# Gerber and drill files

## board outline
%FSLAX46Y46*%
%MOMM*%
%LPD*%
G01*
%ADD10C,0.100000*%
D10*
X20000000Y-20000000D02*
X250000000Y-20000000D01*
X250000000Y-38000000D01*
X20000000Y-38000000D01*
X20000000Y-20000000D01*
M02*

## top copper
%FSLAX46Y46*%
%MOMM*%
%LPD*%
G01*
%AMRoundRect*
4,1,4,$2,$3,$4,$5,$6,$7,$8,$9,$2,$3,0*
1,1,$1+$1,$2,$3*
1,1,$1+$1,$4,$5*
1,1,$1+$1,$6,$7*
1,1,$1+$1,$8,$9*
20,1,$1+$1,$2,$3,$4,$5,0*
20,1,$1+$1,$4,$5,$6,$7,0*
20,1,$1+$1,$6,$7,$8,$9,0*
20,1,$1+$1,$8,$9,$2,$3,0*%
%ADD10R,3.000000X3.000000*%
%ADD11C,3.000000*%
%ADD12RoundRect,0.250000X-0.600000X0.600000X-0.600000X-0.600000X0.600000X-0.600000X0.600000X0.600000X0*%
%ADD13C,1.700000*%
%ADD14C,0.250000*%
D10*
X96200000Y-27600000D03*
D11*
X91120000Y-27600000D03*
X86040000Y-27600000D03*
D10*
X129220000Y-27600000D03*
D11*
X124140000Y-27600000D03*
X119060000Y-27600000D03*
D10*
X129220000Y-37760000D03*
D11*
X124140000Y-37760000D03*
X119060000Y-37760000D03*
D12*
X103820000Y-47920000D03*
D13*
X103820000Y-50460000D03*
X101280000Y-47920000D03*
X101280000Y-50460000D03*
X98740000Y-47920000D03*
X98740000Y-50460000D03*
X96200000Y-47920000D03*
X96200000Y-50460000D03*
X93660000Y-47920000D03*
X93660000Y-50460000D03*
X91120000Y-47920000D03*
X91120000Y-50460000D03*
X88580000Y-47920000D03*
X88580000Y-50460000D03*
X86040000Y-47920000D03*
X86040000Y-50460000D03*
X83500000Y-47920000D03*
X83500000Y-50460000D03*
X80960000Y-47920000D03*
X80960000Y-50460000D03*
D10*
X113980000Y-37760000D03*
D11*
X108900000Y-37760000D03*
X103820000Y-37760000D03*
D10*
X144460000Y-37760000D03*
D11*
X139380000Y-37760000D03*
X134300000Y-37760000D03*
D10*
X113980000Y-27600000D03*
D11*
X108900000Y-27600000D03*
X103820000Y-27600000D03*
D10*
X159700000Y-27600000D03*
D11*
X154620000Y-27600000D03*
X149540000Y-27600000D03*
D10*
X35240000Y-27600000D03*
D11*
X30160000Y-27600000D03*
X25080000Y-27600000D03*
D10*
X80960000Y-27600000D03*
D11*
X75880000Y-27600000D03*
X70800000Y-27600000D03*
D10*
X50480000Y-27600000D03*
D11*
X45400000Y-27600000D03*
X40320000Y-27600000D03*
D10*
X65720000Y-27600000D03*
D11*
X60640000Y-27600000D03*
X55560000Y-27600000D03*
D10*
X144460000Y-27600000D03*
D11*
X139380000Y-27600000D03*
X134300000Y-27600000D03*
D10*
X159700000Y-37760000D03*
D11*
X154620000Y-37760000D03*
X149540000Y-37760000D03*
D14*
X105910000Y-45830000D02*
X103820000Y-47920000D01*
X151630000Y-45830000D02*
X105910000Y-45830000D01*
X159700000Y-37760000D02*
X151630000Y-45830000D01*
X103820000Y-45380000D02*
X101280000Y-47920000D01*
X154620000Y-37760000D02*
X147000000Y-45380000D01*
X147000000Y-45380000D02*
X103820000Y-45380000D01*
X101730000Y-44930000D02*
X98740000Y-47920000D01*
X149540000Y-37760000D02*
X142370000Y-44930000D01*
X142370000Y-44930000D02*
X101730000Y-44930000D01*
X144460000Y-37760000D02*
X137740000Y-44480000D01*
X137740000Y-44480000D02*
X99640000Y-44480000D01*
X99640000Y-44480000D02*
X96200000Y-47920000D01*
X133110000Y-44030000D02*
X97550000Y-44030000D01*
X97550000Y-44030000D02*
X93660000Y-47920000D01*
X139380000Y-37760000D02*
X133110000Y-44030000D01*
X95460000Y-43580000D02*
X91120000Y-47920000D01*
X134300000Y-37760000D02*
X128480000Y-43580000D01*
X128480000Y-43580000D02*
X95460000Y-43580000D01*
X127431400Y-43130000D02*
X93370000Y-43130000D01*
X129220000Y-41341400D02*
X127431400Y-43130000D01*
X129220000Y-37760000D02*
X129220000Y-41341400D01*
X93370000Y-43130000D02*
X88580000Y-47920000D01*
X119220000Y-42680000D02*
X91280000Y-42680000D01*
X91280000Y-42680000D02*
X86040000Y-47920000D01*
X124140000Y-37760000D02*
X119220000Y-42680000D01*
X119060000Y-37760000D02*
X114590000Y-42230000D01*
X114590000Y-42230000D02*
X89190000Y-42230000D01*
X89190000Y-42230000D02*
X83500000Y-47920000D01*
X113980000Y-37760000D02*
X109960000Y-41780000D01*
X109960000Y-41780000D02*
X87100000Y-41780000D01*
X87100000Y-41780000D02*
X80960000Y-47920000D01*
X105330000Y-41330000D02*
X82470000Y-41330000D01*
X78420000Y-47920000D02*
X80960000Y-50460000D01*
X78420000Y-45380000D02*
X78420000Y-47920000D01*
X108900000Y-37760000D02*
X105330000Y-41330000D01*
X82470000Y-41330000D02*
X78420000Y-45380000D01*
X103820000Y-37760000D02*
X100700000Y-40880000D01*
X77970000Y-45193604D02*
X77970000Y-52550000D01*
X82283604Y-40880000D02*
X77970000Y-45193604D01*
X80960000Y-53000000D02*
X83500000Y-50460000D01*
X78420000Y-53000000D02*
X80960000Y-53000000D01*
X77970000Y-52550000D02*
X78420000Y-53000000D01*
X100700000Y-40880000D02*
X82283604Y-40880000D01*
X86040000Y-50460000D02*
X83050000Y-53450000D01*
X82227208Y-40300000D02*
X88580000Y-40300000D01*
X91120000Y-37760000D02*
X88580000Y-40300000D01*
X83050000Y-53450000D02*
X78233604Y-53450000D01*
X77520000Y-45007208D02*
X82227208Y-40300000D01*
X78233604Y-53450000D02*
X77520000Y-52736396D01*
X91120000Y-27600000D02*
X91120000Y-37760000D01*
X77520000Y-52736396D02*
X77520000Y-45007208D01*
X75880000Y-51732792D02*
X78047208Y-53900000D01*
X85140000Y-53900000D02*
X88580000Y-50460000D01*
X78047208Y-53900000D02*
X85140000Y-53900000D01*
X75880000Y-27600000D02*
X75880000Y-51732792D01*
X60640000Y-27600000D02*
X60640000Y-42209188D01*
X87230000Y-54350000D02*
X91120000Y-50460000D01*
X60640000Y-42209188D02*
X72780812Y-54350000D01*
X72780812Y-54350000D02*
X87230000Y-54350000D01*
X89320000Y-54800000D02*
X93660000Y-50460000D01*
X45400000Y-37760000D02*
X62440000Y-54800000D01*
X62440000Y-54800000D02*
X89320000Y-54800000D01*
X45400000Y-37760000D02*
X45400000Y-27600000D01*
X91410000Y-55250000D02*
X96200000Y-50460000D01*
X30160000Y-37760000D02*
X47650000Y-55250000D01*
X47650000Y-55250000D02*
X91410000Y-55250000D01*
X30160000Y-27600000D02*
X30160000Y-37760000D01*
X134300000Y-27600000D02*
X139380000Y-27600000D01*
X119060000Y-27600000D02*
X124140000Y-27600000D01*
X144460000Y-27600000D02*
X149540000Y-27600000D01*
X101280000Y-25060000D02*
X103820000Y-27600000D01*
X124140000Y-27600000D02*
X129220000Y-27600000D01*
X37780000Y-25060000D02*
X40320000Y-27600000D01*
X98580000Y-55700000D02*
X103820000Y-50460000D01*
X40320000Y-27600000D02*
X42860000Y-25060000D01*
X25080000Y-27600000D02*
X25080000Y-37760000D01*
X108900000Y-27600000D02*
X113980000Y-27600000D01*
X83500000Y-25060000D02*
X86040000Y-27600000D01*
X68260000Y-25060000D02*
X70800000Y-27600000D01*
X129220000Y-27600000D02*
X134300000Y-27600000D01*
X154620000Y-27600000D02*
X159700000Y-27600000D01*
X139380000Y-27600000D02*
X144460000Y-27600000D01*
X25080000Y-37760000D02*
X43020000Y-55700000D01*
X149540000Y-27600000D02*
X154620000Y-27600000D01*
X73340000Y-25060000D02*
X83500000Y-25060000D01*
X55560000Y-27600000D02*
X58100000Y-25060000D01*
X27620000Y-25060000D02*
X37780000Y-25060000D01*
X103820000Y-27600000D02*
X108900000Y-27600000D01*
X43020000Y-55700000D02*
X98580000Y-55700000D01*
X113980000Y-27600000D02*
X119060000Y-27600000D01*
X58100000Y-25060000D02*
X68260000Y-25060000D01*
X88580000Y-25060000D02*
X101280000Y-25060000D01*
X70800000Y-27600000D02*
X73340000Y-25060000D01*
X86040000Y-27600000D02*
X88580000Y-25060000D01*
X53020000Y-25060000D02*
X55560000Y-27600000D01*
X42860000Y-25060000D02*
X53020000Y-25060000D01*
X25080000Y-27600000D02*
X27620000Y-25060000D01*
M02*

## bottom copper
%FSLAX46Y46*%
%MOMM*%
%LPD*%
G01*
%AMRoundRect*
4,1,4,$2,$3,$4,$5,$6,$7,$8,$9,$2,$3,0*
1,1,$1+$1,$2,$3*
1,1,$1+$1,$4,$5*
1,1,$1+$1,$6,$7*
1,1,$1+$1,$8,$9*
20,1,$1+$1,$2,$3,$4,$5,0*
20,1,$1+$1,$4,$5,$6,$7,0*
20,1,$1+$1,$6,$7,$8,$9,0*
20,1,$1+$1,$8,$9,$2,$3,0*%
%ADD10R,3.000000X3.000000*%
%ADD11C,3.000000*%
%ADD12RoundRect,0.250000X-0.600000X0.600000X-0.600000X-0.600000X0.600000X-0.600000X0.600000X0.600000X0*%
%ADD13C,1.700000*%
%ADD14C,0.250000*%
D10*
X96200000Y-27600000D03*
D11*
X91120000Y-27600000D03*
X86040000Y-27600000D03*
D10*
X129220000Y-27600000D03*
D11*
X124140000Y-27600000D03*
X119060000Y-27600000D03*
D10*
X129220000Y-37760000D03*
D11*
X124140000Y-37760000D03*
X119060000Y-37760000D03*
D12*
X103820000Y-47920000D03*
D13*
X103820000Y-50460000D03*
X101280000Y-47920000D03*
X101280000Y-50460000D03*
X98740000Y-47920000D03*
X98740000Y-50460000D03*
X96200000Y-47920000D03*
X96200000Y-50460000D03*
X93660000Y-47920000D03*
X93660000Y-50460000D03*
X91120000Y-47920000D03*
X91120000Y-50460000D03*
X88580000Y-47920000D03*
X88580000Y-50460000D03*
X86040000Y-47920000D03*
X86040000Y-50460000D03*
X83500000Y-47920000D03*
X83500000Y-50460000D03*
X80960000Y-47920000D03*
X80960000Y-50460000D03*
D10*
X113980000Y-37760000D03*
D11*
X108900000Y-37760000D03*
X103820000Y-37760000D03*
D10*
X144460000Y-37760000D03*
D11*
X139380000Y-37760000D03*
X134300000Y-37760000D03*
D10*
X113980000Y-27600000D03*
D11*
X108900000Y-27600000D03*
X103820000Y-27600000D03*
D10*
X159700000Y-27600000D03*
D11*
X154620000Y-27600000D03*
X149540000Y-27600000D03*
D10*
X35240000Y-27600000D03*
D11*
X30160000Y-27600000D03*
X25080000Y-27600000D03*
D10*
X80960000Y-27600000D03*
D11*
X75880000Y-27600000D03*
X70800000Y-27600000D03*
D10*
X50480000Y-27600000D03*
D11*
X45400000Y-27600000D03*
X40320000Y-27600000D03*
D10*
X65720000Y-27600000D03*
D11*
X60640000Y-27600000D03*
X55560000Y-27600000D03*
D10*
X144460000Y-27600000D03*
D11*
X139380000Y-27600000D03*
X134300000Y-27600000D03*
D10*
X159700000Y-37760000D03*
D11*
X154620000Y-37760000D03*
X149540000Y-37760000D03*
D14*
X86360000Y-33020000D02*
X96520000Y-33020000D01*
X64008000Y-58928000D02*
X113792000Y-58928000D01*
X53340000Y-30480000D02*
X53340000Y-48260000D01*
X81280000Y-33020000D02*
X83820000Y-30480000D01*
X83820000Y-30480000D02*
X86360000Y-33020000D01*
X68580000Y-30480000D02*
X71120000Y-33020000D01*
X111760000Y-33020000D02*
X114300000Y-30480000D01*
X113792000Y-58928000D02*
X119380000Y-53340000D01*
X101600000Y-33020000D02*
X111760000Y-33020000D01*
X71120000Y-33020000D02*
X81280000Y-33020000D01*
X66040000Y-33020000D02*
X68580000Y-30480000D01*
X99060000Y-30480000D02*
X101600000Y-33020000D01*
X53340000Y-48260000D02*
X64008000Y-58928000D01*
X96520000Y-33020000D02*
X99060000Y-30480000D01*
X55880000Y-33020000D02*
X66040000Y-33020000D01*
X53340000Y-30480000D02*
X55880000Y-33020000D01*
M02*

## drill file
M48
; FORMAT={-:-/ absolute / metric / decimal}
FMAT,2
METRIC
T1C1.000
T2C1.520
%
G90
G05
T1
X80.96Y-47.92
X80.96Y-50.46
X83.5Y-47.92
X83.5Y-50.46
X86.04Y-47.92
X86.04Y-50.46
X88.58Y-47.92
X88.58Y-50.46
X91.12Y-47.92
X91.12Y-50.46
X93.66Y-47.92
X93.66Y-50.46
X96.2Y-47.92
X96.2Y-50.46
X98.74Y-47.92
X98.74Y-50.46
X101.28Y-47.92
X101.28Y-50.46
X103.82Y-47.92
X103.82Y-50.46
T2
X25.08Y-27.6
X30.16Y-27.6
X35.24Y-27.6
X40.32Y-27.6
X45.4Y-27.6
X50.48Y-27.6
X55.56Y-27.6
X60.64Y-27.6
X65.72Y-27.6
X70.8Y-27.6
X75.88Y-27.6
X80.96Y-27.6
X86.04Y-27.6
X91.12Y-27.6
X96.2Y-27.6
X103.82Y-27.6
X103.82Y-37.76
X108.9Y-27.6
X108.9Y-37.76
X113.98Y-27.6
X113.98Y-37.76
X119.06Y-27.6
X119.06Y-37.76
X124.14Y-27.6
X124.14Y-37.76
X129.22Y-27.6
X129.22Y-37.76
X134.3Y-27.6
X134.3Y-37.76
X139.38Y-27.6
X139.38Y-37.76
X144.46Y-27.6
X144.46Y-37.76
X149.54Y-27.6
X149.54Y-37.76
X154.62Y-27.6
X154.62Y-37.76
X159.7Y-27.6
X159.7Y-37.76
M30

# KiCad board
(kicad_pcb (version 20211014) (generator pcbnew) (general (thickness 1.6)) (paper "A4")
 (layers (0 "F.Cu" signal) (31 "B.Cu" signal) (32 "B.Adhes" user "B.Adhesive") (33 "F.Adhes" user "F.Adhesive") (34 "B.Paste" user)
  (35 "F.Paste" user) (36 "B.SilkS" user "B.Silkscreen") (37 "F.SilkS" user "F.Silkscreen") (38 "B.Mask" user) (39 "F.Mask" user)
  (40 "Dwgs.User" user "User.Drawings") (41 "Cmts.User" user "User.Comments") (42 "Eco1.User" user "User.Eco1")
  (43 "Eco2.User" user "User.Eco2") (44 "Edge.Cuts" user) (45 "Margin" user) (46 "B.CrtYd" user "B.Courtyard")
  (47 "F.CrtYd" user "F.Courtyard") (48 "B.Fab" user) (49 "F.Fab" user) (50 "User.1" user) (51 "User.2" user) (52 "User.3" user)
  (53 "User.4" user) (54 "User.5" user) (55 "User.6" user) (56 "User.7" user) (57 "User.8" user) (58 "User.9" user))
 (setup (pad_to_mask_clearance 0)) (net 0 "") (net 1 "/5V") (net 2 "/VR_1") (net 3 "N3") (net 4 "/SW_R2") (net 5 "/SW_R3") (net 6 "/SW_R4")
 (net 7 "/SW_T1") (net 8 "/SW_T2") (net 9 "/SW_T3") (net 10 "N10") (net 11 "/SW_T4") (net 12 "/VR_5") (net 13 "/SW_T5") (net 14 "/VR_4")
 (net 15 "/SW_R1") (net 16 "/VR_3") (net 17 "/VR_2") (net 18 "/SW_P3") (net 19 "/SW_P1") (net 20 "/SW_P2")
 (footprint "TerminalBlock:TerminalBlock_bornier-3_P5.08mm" (layer "F.Cu") (at 96.2 27.6 180)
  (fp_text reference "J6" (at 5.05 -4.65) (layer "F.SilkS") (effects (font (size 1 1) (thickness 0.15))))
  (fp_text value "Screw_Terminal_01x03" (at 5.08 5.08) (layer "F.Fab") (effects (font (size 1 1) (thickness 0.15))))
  (pad "1" thru_hole rect (at 0 0 180) (size 3 3) (drill 1.52) (layers *.Cu *.Mask) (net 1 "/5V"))
  (pad "2" thru_hole circle (at 5.08 0 180) (size 3 3) (drill 1.52) (layers *.Cu *.Mask) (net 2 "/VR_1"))
  (pad "3" thru_hole circle (at 10.16 0 180) (size 3 3) (drill 1.52) (layers *.Cu *.Mask) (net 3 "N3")))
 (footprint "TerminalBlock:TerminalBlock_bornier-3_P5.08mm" (layer "F.Cu") (at 129.22 27.6 180)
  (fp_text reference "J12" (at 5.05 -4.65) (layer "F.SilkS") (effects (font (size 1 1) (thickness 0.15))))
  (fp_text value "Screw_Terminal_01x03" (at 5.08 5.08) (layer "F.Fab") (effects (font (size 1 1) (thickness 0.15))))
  (pad "1" thru_hole rect (at 0 0 180) (size 3 3) (drill 1.52) (layers *.Cu *.Mask) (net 3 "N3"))
  (pad "2" thru_hole circle (at 5.08 0 180) (size 3 3) (drill 1.52) (layers *.Cu *.Mask) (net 3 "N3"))
  (pad "3" thru_hole circle (at 10.16 0 180) (size 3 3) (drill 1.52) (layers *.Cu *.Mask) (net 3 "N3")))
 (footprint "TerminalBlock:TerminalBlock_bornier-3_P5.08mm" (layer "F.Cu") (at 129.22 37.76 180)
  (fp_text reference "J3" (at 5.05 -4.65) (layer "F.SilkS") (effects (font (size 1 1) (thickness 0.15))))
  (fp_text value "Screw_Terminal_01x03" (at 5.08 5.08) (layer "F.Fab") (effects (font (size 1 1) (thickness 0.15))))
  (pad "1" thru_hole rect (at 0 0 180) (size 3 3) (drill 1.52) (layers *.Cu *.Mask) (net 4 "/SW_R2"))
  (pad "2" thru_hole circle (at 5.08 0 180) (size 3 3) (drill 1.52) (layers *.Cu *.Mask) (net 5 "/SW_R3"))
  (pad "3" thru_hole circle (at 10.16 0 180) (size 3 3) (drill 1.52) (layers *.Cu *.Mask) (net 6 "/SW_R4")))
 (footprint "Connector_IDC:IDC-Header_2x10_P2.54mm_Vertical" (layer "F.Cu") (at 103.82 47.92 -90)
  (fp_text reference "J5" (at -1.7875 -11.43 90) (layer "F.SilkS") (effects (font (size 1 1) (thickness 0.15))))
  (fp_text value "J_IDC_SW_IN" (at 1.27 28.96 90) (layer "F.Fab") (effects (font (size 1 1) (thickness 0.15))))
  (pad "1" thru_hole roundrect (at 0 0 270) (size 1.7 1.7) (drill 1) (layers *.Cu *.Mask) (roundrect_rratio 0.147059) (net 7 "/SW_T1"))
  (pad "2" thru_hole circle (at 2.54 0 270) (size 1.7 1.7) (drill 1) (layers *.Cu *.Mask) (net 3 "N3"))
  (pad "3" thru_hole circle (at 0 2.54 270) (size 1.7 1.7) (drill 1) (layers *.Cu *.Mask) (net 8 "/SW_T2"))
  (pad "4" thru_hole circle (at 2.54 2.54 270) (size 1.7 1.7) (drill 1) (layers *.Cu *.Mask) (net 1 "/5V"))
  (pad "5" thru_hole circle (at 0 5.08 270) (size 1.7 1.7) (drill 1) (layers *.Cu *.Mask) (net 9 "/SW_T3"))
  (pad "6" thru_hole circle (at 2.54 5.08 270) (size 1.7 1.7) (drill 1) (layers *.Cu *.Mask) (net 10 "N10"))
  (pad "7" thru_hole circle (at 0 7.62 270) (size 1.7 1.7) (drill 1) (layers *.Cu *.Mask) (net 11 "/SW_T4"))
  (pad "8" thru_hole circle (at 2.54 7.62 270) (size 1.7 1.7) (drill 1) (layers *.Cu *.Mask) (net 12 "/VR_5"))
  (pad "9" thru_hole circle (at 0 10.16 270) (size 1.7 1.7) (drill 1) (layers *.Cu *.Mask) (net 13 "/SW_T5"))
  (pad "10" thru_hole circle (at 2.54 10.16 270) (size 1.7 1.7) (drill 1) (layers *.Cu *.Mask) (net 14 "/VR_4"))
  (pad "11" thru_hole circle (at 0 12.7 270) (size 1.7 1.7) (drill 1) (layers *.Cu *.Mask) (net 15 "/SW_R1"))
  (pad "12" thru_hole circle (at 2.54 12.7 270) (size 1.7 1.7) (drill 1) (layers *.Cu *.Mask) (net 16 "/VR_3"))
  (pad "13" thru_hole circle (at 0 15.24 270) (size 1.7 1.7) (drill 1) (layers *.Cu *.Mask) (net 4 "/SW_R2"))
  (pad "14" thru_hole circle (at 2.54 15.24 270) (size 1.7 1.7) (drill 1) (layers *.Cu *.Mask) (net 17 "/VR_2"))
  (pad "15" thru_hole circle (at 0 17.78 270) (size 1.7 1.7) (drill 1) (layers *.Cu *.Mask) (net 5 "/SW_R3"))
  (pad "16" thru_hole circle (at 2.54 17.78 270) (size 1.7 1.7) (drill 1) (layers *.Cu *.Mask) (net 2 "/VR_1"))
  (pad "17" thru_hole circle (at 0 20.32 270) (size 1.7 1.7) (drill 1) (layers *.Cu *.Mask) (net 6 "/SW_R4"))
  (pad "18" thru_hole circle (at 2.54 20.32 270) (size 1.7 1.7) (drill 1) (layers *.Cu *.Mask) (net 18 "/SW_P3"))
  (pad "19" thru_hole circle (at 0 22.86 270) (size 1.7 1.7) (drill 1) (layers *.Cu *.Mask) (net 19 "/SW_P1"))
  (pad "20" thru_hole circle (at 2.54 22.86 270) (size 1.7 1.7) (drill 1) (layers *.Cu *.Mask) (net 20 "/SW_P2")))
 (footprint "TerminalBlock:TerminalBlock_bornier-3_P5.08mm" (layer "F.Cu") (at 113.98 37.76 180)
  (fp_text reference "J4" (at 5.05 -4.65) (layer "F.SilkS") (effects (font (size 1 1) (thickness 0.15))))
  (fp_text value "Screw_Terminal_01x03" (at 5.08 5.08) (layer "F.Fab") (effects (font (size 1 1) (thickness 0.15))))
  (pad "1" thru_hole rect (at 0 0 180) (size 3 3) (drill 1.52) (layers *.Cu *.Mask) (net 19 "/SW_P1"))
  (pad "2" thru_hole circle (at 5.08 0 180) (size 3 3) (drill 1.52) (layers *.Cu *.Mask) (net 20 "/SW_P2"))
  (pad "3" thru_hole circle (at 10.16 0 180) (size 3 3) (drill 1.52) (layers *.Cu *.Mask) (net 18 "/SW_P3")))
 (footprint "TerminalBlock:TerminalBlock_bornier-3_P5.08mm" (layer "F.Cu") (at 144.46 37.76 180)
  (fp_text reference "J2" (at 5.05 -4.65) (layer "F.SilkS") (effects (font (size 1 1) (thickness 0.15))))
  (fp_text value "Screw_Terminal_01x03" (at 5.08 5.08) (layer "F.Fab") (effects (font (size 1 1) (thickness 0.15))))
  (pad "1" thru_hole rect (at 0 0 180) (size 3 3) (drill 1.52) (layers *.Cu *.Mask) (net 11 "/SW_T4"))
  (pad "2" thru_hole circle (at 5.08 0 180) (size 3 3) (drill 1.52) (layers *.Cu *.Mask) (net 13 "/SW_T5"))
  (pad "3" thru_hole circle (at 10.16 0 180) (size 3 3) (drill 1.52) (layers *.Cu *.Mask) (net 15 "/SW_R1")))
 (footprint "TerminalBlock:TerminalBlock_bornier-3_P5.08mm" (layer "F.Cu") (at 113.98 27.6 180)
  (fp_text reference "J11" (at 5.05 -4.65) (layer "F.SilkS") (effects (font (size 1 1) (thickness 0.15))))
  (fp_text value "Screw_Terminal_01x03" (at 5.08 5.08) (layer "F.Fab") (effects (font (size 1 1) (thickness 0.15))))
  (pad "1" thru_hole rect (at 0 0 180) (size 3 3) (drill 1.52) (layers *.Cu *.Mask) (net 3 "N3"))
  (pad "2" thru_hole circle (at 5.08 0 180) (size 3 3) (drill 1.52) (layers *.Cu *.Mask) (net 3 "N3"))
  (pad "3" thru_hole circle (at 10.16 0 180) (size 3 3) (drill 1.52) (layers *.Cu *.Mask) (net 3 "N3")))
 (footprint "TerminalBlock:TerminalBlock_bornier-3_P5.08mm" (layer "F.Cu") (at 159.7 27.6 180)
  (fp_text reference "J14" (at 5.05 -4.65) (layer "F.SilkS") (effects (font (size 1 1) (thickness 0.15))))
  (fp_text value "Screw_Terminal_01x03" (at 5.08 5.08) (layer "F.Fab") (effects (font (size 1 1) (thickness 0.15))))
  (pad "1" thru_hole rect (at 0 0 180) (size 3 3) (drill 1.52) (layers *.Cu *.Mask) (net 3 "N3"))
  (pad "2" thru_hole circle (at 5.08 0 180) (size 3 3) (drill 1.52) (layers *.Cu *.Mask) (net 3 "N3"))
  (pad "3" thru_hole circle (at 10.16 0 180) (size 3 3) (drill 1.52) (layers *.Cu *.Mask) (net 3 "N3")))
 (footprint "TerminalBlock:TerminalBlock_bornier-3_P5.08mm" (layer "F.Cu") (at 35.24 27.6 180)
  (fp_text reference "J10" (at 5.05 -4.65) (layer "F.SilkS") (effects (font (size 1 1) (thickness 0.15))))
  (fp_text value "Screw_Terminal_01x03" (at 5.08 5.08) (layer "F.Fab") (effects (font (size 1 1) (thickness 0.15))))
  (pad "1" thru_hole rect (at 0 0 180) (size 3 3) (drill 1.52) (layers *.Cu *.Mask) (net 1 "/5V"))
  (pad "2" thru_hole circle (at 5.08 0 180) (size 3 3) (drill 1.52) (layers *.Cu *.Mask) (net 12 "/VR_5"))
  (pad "3" thru_hole circle (at 10.16 0 180) (size 3 3) (drill 1.52) (layers *.Cu *.Mask) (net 3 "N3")))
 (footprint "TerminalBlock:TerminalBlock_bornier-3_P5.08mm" (layer "F.Cu") (at 80.96 27.6 180)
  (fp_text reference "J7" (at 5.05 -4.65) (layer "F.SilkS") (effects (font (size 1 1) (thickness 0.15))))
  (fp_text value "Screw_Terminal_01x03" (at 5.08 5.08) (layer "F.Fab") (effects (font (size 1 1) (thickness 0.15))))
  (pad "1" thru_hole rect (at 0 0 180) (size 3 3) (drill 1.52) (layers *.Cu *.Mask) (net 1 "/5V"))
  (pad "2" thru_hole circle (at 5.08 0 180) (size 3 3) (drill 1.52) (layers *.Cu *.Mask) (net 17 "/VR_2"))
  (pad "3" thru_hole circle (at 10.16 0 180) (size 3 3) (drill 1.52) (layers *.Cu *.Mask) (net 3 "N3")))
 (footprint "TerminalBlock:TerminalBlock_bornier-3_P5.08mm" (layer "F.Cu") (at 50.48 27.6 180)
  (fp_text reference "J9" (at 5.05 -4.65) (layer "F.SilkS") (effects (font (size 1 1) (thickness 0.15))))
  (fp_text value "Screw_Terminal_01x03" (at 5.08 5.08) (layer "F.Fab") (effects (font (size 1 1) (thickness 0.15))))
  (pad "1" thru_hole rect (at 0 0 180) (size 3 3) (drill 1.52) (layers *.Cu *.Mask) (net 1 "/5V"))
  (pad "2" thru_hole circle (at 5.08 0 180) (size 3 3) (drill 1.52) (layers *.Cu *.Mask) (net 14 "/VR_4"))
  (pad "3" thru_hole circle (at 10.16 0 180) (size 3 3) (drill 1.52) (layers *.Cu *.Mask) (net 3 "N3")))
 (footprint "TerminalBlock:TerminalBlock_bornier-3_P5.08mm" (layer "F.Cu") (at 65.72 27.6 180)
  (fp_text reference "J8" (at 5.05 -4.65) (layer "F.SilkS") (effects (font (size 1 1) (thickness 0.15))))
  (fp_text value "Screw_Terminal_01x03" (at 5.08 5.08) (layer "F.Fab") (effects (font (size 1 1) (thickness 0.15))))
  (pad "1" thru_hole rect (at 0 0 180) (size 3 3) (drill 1.52) (layers *.Cu *.Mask) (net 1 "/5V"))
  (pad "2" thru_hole circle (at 5.08 0 180) (size 3 3) (drill 1.52) (layers *.Cu *.Mask) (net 16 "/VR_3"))
  (pad "3" thru_hole circle (at 10.16 0 180) (size 3 3) (drill 1.52) (layers *.Cu *.Mask) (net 3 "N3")))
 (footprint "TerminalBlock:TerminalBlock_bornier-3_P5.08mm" (layer "F.Cu") (at 144.46 27.6 180)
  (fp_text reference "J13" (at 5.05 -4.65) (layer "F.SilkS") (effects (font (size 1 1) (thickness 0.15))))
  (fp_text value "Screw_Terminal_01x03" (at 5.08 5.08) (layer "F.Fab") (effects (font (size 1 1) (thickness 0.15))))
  (pad "1" thru_hole rect (at 0 0 180) (size 3 3) (drill 1.52) (layers *.Cu *.Mask) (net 3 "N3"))
  (pad "2" thru_hole circle (at 5.08 0 180) (size 3 3) (drill 1.52) (layers *.Cu *.Mask) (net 3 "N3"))
  (pad "3" thru_hole circle (at 10.16 0 180) (size 3 3) (drill 1.52) (layers *.Cu *.Mask) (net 3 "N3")))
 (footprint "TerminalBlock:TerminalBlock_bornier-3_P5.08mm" (layer "F.Cu") (at 159.7 37.76 180)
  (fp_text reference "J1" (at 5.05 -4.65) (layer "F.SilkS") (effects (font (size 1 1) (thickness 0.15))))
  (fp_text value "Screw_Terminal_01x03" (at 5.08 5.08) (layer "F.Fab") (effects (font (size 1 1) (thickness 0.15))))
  (pad "1" thru_hole rect (at 0 0 180) (size 3 3) (drill 1.52) (layers *.Cu *.Mask) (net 7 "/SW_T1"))
  (pad "2" thru_hole circle (at 5.08 0 180) (size 3 3) (drill 1.52) (layers *.Cu *.Mask) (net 8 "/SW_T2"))
  (pad "3" thru_hole circle (at 10.16 0 180) (size 3 3) (drill 1.52) (layers *.Cu *.Mask) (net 9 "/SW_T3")))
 (gr_rect (start 20 20) (end 250 38) (layer "Edge.Cuts") (width 0.1) (fill none))
 (segment (start 105.91 45.83) (end 103.82 47.92) (width 0.25) (layer "F.Cu") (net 7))
 (segment (start 151.63 45.83) (end 105.91 45.83) (width 0.25) (layer "F.Cu") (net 7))
 (segment (start 159.7 37.76) (end 151.63 45.83) (width 0.25) (layer "F.Cu") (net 7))
 (segment (start 103.82 45.38) (end 101.28 47.92) (width 0.25) (layer "F.Cu") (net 8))
 (segment (start 154.62 37.76) (end 147 45.38) (width 0.25) (layer "F.Cu") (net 8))
 (segment (start 147 45.38) (end 103.82 45.38) (width 0.25) (layer "F.Cu") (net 8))
 (segment (start 101.73 44.93) (end 98.74 47.92) (width 0.25) (layer "F.Cu") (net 9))
 (segment (start 149.54 37.76) (end 142.37 44.93) (width 0.25) (layer "F.Cu") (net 9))
 (segment (start 142.37 44.93) (end 101.73 44.93) (width 0.25) (layer "F.Cu") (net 9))
 (segment (start 144.46 37.76) (end 137.74 44.48) (width 0.25) (layer "F.Cu") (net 11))
 (segment (start 137.74 44.48) (end 99.64 44.48) (width 0.25) (layer "F.Cu") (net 11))
 (segment (start 99.64 44.48) (end 96.2 47.92) (width 0.25) (layer "F.Cu") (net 11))
 (segment (start 133.11 44.03) (end 97.55 44.03) (width 0.25) (layer "F.Cu") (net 13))
 (segment (start 97.55 44.03) (end 93.66 47.92) (width 0.25) (layer "F.Cu") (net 13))
 (segment (start 139.38 37.76) (end 133.11 44.03) (width 0.25) (layer "F.Cu") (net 13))
 (segment (start 95.46 43.58) (end 91.12 47.92) (width 0.25) (layer "F.Cu") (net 15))
 (segment (start 134.3 37.76) (end 128.48 43.58) (width 0.25) (layer "F.Cu") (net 15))
 (segment (start 128.48 43.58) (end 95.46 43.58) (width 0.25) (layer "F.Cu") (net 15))
 (segment (start 127.4314 43.13) (end 93.37 43.13) (width 0.25) (layer "F.Cu") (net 4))
 (segment (start 129.22 41.3414) (end 127.4314 43.13) (width 0.25) (layer "F.Cu") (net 4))
 (segment (start 129.22 37.76) (end 129.22 41.3414) (width 0.25) (layer "F.Cu") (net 4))
 (segment (start 93.37 43.13) (end 88.58 47.92) (width 0.25) (layer "F.Cu") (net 4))
 (segment (start 119.22 42.68) (end 91.28 42.68) (width 0.25) (layer "F.Cu") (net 5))
 (segment (start 91.28 42.68) (end 86.04 47.92) (width 0.25) (layer "F.Cu") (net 5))
 (segment (start 124.14 37.76) (end 119.22 42.68) (width 0.25) (layer "F.Cu") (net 5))
 (segment (start 119.06 37.76) (end 114.59 42.23) (width 0.25) (layer "F.Cu") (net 6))
 (segment (start 114.59 42.23) (end 89.19 42.23) (width 0.25) (layer "F.Cu") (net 6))
 (segment (start 89.19 42.23) (end 83.5 47.92) (width 0.25) (layer "F.Cu") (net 6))
 (segment (start 113.98 37.76) (end 109.96 41.78) (width 0.25) (layer "F.Cu") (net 19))
 (segment (start 109.96 41.78) (end 87.1 41.78) (width 0.25) (layer "F.Cu") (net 19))
 (segment (start 87.1 41.78) (end 80.96 47.92) (width 0.25) (layer "F.Cu") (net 19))
 (segment (start 105.33 41.33) (end 82.47 41.33) (width 0.25) (layer "F.Cu") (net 20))
 (segment (start 78.42 47.92) (end 80.96 50.46) (width 0.25) (layer "F.Cu") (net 20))
 (segment (start 78.42 45.38) (end 78.42 47.92) (width 0.25) (layer "F.Cu") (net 20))
 (segment (start 108.9 37.76) (end 105.33 41.33) (width 0.25) (layer "F.Cu") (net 20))
 (segment (start 82.47 41.33) (end 78.42 45.38) (width 0.25) (layer "F.Cu") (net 20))
 (segment (start 103.82 37.76) (end 100.7 40.88) (width 0.25) (layer "F.Cu") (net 18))
 (segment (start 77.97 45.193604) (end 77.97 52.55) (width 0.25) (layer "F.Cu") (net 18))
 (segment (start 82.283604 40.88) (end 77.97 45.193604) (width 0.25) (layer "F.Cu") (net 18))
 (segment (start 80.96 53) (end 83.5 50.46) (width 0.25) (layer "F.Cu") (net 18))
 (segment (start 78.42 53) (end 80.96 53) (width 0.25) (layer "F.Cu") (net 18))
 (segment (start 77.97 52.55) (end 78.42 53) (width 0.25) (layer "F.Cu") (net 18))
 (segment (start 100.7 40.88) (end 82.283604 40.88) (width 0.25) (layer "F.Cu") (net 18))
 (segment (start 86.04 50.46) (end 83.05 53.45) (width 0.25) (layer "F.Cu") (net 2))
 (segment (start 82.227208 40.3) (end 88.58 40.3) (width 0.25) (layer "F.Cu") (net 2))
 (segment (start 91.12 37.76) (end 88.58 40.3) (width 0.25) (layer "F.Cu") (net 2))
 (segment (start 83.05 53.45) (end 78.233604 53.45) (width 0.25) (layer "F.Cu") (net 2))
 (segment (start 77.52 45.007208) (end 82.227208 40.3) (width 0.25) (layer "F.Cu") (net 2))
 (segment (start 78.233604 53.45) (end 77.52 52.736396) (width 0.25) (layer "F.Cu") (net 2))
 (segment (start 91.12 27.6) (end 91.12 37.76) (width 0.25) (layer "F.Cu") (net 2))
 (segment (start 77.52 52.736396) (end 77.52 45.007208) (width 0.25) (layer "F.Cu") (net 2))
 (segment (start 75.88 51.732792) (end 78.047208 53.9) (width 0.25) (layer "F.Cu") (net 17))
 (segment (start 85.14 53.9) (end 88.58 50.46) (width 0.25) (layer "F.Cu") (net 17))
 (segment (start 78.047208 53.9) (end 85.14 53.9) (width 0.25) (layer "F.Cu") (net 17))
 (segment (start 75.88 27.6) (end 75.88 51.732792) (width 0.25) (layer "F.Cu") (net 17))
 (segment (start 60.64 27.6) (end 60.64 42.209188) (width 0.25) (layer "F.Cu") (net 16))
 (segment (start 87.23 54.35) (end 91.12 50.46) (width 0.25) (layer "F.Cu") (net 16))
 (segment (start 60.64 42.209188) (end 72.780812 54.35) (width 0.25) (layer "F.Cu") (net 16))
 (segment (start 72.780812 54.35) (end 87.23 54.35) (width 0.25) (layer "F.Cu") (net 16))
 (segment (start 89.32 54.8) (end 93.66 50.46) (width 0.25) (layer "F.Cu") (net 14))
 (segment (start 45.4 37.76) (end 62.44 54.8) (width 0.25) (layer "F.Cu") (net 14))
 (segment (start 62.44 54.8) (end 89.32 54.8) (width 0.25) (layer "F.Cu") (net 14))
 (segment (start 45.4 37.76) (end 45.4 27.6) (width 0.25) (layer "F.Cu") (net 14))
 (segment (start 91.41 55.25) (end 96.2 50.46) (width 0.25) (layer "F.Cu") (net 12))
 (segment (start 30.16 37.76) (end 47.65 55.25) (width 0.25) (layer "F.Cu") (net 12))
 (segment (start 47.65 55.25) (end 91.41 55.25) (width 0.25) (layer "F.Cu") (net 12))
 (segment (start 30.16 27.6) (end 30.16 37.76) (width 0.25) (layer "F.Cu") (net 12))
 (segment (start 134.3 27.6) (end 139.38 27.6) (width 0.25) (layer "F.Cu") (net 3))
 (segment (start 119.06 27.6) (end 124.14 27.6) (width 0.25) (layer "F.Cu") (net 3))
 (segment (start 144.46 27.6) (end 149.54 27.6) (width 0.25) (layer "F.Cu") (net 3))
 (segment (start 101.28 25.06) (end 103.82 27.6) (width 0.25) (layer "F.Cu") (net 3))
 (segment (start 124.14 27.6) (end 129.22 27.6) (width 0.25) (layer "F.Cu") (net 3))
 (segment (start 37.78 25.06) (end 40.32 27.6) (width 0.25) (layer "F.Cu") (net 3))
 (segment (start 98.58 55.7) (end 103.82 50.46) (width 0.25) (layer "F.Cu") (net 3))
 (segment (start 40.32 27.6) (end 42.86 25.06) (width 0.25) (layer "F.Cu") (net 3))
 (segment (start 25.08 27.6) (end 25.08 37.76) (width 0.25) (layer "F.Cu") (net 3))
 (segment (start 108.9 27.6) (end 113.98 27.6) (width 0.25) (layer "F.Cu") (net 3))
 (segment (start 83.5 25.06) (end 86.04 27.6) (width 0.25) (layer "F.Cu") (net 3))
 (segment (start 68.26 25.06) (end 70.8 27.6) (width 0.25) (layer "F.Cu") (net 3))
 (segment (start 129.22 27.6) (end 134.3 27.6) (width 0.25) (layer "F.Cu") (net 3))
 (segment (start 154.62 27.6) (end 159.7 27.6) (width 0.25) (layer "F.Cu") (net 3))
 (segment (start 139.38 27.6) (end 144.46 27.6) (width 0.25) (layer "F.Cu") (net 3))
 (segment (start 25.08 37.76) (end 43.02 55.7) (width 0.25) (layer "F.Cu") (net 3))
 (segment (start 149.54 27.6) (end 154.62 27.6) (width 0.25) (layer "F.Cu") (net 3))
 (segment (start 73.34 25.06) (end 83.5 25.06) (width 0.25) (layer "F.Cu") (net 3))
 (segment (start 55.56 27.6) (end 58.1 25.06) (width 0.25) (layer "F.Cu") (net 3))
 (segment (start 27.62 25.06) (end 37.78 25.06) (width 0.25) (layer "F.Cu") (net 3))
 (segment (start 103.82 27.6) (end 108.9 27.6) (width 0.25) (layer "F.Cu") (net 3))
 (segment (start 43.02 55.7) (end 98.58 55.7) (width 0.25) (layer "F.Cu") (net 3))
 (segment (start 113.98 27.6) (end 119.06 27.6) (width 0.25) (layer "F.Cu") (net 3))
 (segment (start 58.1 25.06) (end 68.26 25.06) (width 0.25) (layer "F.Cu") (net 3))
 (segment (start 88.58 25.06) (end 101.28 25.06) (width 0.25) (layer "F.Cu") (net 3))
 (segment (start 70.8 27.6) (end 73.34 25.06) (width 0.25) (layer "F.Cu") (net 3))
 (segment (start 86.04 27.6) (end 88.58 25.06) (width 0.25) (layer "F.Cu") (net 3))
 (segment (start 53.02 25.06) (end 55.56 27.6) (width 0.25) (layer "F.Cu") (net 3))
 (segment (start 42.86 25.06) (end 53.02 25.06) (width 0.25) (layer "F.Cu") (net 3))
 (segment (start 25.08 27.6) (end 27.62 25.06) (width 0.25) (layer "F.Cu") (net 3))
 (segment (start 86.36 33.02) (end 96.52 33.02) (width 0.25) (layer "B.Cu") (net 1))
 (segment (start 64.008 58.928) (end 113.792 58.928) (width 0.25) (layer "B.Cu") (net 1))
 (segment (start 53.34 30.48) (end 53.34 48.26) (width 0.25) (layer "B.Cu") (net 1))
 (segment (start 81.28 33.02) (end 83.82 30.48) (width 0.25) (layer "B.Cu") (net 1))
 (segment (start 83.82 30.48) (end 86.36 33.02) (width 0.25) (layer "B.Cu") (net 1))
 (segment (start 68.58 30.48) (end 71.12 33.02) (width 0.25) (layer "B.Cu") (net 1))
 (segment (start 111.76 33.02) (end 114.3 30.48) (width 0.25) (layer "B.Cu") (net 1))
 (segment (start 113.792 58.928) (end 119.38 53.34) (width 0.25) (layer "B.Cu") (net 1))
 (segment (start 101.6 33.02) (end 111.76 33.02) (width 0.25) (layer "B.Cu") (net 1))
 (segment (start 71.12 33.02) (end 81.28 33.02) (width 0.25) (layer "B.Cu") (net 1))
 (segment (start 66.04 33.02) (end 68.58 30.48) (width 0.25) (layer "B.Cu") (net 1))
 (segment (start 99.06 30.48) (end 101.6 33.02) (width 0.25) (layer "B.Cu") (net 1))
 (segment (start 53.34 48.26) (end 64.008 58.928) (width 0.25) (layer "B.Cu") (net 1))
 (segment (start 96.52 33.02) (end 99.06 30.48) (width 0.25) (layer "B.Cu") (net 1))
 (segment (start 55.88 33.02) (end 66.04 33.02) (width 0.25) (layer "B.Cu") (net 1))
 (segment (start 53.34 30.48) (end 55.88 33.02) (width 0.25) (layer "B.Cu") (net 1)))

